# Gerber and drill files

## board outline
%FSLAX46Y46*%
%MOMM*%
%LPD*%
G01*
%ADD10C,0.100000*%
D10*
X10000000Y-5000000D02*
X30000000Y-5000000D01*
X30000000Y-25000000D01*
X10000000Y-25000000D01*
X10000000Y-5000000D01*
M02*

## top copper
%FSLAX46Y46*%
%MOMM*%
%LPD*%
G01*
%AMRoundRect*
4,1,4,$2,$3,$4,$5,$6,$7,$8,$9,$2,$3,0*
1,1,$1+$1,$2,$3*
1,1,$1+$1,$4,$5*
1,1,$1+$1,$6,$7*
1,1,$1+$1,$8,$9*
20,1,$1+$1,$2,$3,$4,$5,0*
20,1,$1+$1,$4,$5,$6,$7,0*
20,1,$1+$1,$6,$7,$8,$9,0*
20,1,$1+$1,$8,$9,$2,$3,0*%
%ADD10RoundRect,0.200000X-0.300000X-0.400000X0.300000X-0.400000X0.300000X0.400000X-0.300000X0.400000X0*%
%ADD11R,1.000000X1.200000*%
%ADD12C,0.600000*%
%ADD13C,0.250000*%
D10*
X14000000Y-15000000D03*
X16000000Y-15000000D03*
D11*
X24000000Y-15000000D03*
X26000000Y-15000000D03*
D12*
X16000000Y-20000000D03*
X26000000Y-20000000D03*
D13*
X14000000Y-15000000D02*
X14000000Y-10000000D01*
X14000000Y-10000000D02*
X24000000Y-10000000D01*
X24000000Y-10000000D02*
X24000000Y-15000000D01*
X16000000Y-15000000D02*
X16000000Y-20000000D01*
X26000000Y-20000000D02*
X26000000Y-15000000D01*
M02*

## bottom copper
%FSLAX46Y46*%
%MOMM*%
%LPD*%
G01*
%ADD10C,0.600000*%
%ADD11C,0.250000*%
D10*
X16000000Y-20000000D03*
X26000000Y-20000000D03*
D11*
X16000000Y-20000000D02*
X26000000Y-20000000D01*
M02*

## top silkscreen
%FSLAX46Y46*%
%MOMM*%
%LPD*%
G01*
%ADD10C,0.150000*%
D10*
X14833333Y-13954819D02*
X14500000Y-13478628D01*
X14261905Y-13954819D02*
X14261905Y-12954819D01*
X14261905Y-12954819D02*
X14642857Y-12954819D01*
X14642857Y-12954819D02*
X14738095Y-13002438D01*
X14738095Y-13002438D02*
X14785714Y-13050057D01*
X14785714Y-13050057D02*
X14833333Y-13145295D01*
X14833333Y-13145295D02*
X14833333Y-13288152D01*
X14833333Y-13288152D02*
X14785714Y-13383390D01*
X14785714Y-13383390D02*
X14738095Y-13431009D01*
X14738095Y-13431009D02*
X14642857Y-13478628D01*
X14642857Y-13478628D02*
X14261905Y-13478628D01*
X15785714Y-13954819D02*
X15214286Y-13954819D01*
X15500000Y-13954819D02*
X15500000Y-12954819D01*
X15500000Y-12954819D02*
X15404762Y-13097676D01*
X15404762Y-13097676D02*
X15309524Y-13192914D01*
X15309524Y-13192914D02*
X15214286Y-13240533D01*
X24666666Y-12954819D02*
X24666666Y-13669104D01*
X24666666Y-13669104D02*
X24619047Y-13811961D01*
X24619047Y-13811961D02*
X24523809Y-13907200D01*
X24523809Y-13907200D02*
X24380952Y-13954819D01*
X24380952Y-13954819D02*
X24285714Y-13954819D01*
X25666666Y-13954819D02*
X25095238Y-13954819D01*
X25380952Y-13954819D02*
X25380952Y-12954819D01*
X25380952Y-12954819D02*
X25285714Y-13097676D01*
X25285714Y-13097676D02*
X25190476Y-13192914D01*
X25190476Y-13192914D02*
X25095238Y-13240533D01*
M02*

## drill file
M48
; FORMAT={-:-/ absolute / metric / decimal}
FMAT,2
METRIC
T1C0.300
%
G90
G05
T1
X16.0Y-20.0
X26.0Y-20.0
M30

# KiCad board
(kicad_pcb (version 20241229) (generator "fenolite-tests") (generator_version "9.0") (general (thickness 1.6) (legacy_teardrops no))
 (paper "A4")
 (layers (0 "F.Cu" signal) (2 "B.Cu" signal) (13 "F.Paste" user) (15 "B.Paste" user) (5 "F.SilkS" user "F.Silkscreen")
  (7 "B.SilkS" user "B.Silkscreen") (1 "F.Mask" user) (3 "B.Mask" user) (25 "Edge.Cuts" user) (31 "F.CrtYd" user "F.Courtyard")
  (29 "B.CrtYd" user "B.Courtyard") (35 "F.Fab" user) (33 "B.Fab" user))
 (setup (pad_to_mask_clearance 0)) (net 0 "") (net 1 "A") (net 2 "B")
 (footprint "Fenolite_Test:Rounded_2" (layer "F.Cu") (at 15 15)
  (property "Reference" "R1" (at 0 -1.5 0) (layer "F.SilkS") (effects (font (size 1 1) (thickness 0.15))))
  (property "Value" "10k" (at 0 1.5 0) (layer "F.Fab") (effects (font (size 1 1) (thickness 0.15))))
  (pad "1" smd roundrect (at -1 0) (size 1 1.2) (layers "F.Cu" "F.Paste" "F.Mask") (roundrect_rratio 0.2) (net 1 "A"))
  (pad "2" smd roundrect (at 1 0) (size 1 1.2) (layers "F.Cu" "F.Paste" "F.Mask") (roundrect_rratio 0.2) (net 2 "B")))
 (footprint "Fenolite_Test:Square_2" (layer "F.Cu") (at 25 15)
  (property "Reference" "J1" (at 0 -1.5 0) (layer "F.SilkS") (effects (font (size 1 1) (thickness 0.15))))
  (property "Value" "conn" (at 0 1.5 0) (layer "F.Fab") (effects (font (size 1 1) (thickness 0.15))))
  (pad "1" smd rect (at -1 0) (size 1 1.2) (layers "F.Cu" "F.Paste" "F.Mask") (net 1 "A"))
  (pad "2" smd rect (at 1 0) (size 1 1.2) (layers "F.Cu" "F.Paste" "F.Mask") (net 2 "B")))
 (segment (start 14 15) (end 14 10) (width 0.25) (layer "F.Cu") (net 1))
 (segment (start 14 10) (end 24 10) (width 0.25) (layer "F.Cu") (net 1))
 (segment (start 24 10) (end 24 15) (width 0.25) (layer "F.Cu") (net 1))
 (segment (start 16 15) (end 16 20) (width 0.25) (layer "F.Cu") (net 2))
 (via (at 16 20) (size 0.6) (drill 0.3) (layers "F.Cu" "B.Cu") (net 2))
 (segment (start 16 20) (end 26 20) (width 0.25) (layer "B.Cu") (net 2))
 (via (at 26 20) (size 0.6) (drill 0.3) (layers "F.Cu" "B.Cu") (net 2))
 (segment (start 26 20) (end 26 15) (width 0.25) (layer "F.Cu") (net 2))
 (gr_rect (start 10 5) (end 30 25) (stroke (width 0.1) (type default)) (fill no) (layer "Edge.Cuts")))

